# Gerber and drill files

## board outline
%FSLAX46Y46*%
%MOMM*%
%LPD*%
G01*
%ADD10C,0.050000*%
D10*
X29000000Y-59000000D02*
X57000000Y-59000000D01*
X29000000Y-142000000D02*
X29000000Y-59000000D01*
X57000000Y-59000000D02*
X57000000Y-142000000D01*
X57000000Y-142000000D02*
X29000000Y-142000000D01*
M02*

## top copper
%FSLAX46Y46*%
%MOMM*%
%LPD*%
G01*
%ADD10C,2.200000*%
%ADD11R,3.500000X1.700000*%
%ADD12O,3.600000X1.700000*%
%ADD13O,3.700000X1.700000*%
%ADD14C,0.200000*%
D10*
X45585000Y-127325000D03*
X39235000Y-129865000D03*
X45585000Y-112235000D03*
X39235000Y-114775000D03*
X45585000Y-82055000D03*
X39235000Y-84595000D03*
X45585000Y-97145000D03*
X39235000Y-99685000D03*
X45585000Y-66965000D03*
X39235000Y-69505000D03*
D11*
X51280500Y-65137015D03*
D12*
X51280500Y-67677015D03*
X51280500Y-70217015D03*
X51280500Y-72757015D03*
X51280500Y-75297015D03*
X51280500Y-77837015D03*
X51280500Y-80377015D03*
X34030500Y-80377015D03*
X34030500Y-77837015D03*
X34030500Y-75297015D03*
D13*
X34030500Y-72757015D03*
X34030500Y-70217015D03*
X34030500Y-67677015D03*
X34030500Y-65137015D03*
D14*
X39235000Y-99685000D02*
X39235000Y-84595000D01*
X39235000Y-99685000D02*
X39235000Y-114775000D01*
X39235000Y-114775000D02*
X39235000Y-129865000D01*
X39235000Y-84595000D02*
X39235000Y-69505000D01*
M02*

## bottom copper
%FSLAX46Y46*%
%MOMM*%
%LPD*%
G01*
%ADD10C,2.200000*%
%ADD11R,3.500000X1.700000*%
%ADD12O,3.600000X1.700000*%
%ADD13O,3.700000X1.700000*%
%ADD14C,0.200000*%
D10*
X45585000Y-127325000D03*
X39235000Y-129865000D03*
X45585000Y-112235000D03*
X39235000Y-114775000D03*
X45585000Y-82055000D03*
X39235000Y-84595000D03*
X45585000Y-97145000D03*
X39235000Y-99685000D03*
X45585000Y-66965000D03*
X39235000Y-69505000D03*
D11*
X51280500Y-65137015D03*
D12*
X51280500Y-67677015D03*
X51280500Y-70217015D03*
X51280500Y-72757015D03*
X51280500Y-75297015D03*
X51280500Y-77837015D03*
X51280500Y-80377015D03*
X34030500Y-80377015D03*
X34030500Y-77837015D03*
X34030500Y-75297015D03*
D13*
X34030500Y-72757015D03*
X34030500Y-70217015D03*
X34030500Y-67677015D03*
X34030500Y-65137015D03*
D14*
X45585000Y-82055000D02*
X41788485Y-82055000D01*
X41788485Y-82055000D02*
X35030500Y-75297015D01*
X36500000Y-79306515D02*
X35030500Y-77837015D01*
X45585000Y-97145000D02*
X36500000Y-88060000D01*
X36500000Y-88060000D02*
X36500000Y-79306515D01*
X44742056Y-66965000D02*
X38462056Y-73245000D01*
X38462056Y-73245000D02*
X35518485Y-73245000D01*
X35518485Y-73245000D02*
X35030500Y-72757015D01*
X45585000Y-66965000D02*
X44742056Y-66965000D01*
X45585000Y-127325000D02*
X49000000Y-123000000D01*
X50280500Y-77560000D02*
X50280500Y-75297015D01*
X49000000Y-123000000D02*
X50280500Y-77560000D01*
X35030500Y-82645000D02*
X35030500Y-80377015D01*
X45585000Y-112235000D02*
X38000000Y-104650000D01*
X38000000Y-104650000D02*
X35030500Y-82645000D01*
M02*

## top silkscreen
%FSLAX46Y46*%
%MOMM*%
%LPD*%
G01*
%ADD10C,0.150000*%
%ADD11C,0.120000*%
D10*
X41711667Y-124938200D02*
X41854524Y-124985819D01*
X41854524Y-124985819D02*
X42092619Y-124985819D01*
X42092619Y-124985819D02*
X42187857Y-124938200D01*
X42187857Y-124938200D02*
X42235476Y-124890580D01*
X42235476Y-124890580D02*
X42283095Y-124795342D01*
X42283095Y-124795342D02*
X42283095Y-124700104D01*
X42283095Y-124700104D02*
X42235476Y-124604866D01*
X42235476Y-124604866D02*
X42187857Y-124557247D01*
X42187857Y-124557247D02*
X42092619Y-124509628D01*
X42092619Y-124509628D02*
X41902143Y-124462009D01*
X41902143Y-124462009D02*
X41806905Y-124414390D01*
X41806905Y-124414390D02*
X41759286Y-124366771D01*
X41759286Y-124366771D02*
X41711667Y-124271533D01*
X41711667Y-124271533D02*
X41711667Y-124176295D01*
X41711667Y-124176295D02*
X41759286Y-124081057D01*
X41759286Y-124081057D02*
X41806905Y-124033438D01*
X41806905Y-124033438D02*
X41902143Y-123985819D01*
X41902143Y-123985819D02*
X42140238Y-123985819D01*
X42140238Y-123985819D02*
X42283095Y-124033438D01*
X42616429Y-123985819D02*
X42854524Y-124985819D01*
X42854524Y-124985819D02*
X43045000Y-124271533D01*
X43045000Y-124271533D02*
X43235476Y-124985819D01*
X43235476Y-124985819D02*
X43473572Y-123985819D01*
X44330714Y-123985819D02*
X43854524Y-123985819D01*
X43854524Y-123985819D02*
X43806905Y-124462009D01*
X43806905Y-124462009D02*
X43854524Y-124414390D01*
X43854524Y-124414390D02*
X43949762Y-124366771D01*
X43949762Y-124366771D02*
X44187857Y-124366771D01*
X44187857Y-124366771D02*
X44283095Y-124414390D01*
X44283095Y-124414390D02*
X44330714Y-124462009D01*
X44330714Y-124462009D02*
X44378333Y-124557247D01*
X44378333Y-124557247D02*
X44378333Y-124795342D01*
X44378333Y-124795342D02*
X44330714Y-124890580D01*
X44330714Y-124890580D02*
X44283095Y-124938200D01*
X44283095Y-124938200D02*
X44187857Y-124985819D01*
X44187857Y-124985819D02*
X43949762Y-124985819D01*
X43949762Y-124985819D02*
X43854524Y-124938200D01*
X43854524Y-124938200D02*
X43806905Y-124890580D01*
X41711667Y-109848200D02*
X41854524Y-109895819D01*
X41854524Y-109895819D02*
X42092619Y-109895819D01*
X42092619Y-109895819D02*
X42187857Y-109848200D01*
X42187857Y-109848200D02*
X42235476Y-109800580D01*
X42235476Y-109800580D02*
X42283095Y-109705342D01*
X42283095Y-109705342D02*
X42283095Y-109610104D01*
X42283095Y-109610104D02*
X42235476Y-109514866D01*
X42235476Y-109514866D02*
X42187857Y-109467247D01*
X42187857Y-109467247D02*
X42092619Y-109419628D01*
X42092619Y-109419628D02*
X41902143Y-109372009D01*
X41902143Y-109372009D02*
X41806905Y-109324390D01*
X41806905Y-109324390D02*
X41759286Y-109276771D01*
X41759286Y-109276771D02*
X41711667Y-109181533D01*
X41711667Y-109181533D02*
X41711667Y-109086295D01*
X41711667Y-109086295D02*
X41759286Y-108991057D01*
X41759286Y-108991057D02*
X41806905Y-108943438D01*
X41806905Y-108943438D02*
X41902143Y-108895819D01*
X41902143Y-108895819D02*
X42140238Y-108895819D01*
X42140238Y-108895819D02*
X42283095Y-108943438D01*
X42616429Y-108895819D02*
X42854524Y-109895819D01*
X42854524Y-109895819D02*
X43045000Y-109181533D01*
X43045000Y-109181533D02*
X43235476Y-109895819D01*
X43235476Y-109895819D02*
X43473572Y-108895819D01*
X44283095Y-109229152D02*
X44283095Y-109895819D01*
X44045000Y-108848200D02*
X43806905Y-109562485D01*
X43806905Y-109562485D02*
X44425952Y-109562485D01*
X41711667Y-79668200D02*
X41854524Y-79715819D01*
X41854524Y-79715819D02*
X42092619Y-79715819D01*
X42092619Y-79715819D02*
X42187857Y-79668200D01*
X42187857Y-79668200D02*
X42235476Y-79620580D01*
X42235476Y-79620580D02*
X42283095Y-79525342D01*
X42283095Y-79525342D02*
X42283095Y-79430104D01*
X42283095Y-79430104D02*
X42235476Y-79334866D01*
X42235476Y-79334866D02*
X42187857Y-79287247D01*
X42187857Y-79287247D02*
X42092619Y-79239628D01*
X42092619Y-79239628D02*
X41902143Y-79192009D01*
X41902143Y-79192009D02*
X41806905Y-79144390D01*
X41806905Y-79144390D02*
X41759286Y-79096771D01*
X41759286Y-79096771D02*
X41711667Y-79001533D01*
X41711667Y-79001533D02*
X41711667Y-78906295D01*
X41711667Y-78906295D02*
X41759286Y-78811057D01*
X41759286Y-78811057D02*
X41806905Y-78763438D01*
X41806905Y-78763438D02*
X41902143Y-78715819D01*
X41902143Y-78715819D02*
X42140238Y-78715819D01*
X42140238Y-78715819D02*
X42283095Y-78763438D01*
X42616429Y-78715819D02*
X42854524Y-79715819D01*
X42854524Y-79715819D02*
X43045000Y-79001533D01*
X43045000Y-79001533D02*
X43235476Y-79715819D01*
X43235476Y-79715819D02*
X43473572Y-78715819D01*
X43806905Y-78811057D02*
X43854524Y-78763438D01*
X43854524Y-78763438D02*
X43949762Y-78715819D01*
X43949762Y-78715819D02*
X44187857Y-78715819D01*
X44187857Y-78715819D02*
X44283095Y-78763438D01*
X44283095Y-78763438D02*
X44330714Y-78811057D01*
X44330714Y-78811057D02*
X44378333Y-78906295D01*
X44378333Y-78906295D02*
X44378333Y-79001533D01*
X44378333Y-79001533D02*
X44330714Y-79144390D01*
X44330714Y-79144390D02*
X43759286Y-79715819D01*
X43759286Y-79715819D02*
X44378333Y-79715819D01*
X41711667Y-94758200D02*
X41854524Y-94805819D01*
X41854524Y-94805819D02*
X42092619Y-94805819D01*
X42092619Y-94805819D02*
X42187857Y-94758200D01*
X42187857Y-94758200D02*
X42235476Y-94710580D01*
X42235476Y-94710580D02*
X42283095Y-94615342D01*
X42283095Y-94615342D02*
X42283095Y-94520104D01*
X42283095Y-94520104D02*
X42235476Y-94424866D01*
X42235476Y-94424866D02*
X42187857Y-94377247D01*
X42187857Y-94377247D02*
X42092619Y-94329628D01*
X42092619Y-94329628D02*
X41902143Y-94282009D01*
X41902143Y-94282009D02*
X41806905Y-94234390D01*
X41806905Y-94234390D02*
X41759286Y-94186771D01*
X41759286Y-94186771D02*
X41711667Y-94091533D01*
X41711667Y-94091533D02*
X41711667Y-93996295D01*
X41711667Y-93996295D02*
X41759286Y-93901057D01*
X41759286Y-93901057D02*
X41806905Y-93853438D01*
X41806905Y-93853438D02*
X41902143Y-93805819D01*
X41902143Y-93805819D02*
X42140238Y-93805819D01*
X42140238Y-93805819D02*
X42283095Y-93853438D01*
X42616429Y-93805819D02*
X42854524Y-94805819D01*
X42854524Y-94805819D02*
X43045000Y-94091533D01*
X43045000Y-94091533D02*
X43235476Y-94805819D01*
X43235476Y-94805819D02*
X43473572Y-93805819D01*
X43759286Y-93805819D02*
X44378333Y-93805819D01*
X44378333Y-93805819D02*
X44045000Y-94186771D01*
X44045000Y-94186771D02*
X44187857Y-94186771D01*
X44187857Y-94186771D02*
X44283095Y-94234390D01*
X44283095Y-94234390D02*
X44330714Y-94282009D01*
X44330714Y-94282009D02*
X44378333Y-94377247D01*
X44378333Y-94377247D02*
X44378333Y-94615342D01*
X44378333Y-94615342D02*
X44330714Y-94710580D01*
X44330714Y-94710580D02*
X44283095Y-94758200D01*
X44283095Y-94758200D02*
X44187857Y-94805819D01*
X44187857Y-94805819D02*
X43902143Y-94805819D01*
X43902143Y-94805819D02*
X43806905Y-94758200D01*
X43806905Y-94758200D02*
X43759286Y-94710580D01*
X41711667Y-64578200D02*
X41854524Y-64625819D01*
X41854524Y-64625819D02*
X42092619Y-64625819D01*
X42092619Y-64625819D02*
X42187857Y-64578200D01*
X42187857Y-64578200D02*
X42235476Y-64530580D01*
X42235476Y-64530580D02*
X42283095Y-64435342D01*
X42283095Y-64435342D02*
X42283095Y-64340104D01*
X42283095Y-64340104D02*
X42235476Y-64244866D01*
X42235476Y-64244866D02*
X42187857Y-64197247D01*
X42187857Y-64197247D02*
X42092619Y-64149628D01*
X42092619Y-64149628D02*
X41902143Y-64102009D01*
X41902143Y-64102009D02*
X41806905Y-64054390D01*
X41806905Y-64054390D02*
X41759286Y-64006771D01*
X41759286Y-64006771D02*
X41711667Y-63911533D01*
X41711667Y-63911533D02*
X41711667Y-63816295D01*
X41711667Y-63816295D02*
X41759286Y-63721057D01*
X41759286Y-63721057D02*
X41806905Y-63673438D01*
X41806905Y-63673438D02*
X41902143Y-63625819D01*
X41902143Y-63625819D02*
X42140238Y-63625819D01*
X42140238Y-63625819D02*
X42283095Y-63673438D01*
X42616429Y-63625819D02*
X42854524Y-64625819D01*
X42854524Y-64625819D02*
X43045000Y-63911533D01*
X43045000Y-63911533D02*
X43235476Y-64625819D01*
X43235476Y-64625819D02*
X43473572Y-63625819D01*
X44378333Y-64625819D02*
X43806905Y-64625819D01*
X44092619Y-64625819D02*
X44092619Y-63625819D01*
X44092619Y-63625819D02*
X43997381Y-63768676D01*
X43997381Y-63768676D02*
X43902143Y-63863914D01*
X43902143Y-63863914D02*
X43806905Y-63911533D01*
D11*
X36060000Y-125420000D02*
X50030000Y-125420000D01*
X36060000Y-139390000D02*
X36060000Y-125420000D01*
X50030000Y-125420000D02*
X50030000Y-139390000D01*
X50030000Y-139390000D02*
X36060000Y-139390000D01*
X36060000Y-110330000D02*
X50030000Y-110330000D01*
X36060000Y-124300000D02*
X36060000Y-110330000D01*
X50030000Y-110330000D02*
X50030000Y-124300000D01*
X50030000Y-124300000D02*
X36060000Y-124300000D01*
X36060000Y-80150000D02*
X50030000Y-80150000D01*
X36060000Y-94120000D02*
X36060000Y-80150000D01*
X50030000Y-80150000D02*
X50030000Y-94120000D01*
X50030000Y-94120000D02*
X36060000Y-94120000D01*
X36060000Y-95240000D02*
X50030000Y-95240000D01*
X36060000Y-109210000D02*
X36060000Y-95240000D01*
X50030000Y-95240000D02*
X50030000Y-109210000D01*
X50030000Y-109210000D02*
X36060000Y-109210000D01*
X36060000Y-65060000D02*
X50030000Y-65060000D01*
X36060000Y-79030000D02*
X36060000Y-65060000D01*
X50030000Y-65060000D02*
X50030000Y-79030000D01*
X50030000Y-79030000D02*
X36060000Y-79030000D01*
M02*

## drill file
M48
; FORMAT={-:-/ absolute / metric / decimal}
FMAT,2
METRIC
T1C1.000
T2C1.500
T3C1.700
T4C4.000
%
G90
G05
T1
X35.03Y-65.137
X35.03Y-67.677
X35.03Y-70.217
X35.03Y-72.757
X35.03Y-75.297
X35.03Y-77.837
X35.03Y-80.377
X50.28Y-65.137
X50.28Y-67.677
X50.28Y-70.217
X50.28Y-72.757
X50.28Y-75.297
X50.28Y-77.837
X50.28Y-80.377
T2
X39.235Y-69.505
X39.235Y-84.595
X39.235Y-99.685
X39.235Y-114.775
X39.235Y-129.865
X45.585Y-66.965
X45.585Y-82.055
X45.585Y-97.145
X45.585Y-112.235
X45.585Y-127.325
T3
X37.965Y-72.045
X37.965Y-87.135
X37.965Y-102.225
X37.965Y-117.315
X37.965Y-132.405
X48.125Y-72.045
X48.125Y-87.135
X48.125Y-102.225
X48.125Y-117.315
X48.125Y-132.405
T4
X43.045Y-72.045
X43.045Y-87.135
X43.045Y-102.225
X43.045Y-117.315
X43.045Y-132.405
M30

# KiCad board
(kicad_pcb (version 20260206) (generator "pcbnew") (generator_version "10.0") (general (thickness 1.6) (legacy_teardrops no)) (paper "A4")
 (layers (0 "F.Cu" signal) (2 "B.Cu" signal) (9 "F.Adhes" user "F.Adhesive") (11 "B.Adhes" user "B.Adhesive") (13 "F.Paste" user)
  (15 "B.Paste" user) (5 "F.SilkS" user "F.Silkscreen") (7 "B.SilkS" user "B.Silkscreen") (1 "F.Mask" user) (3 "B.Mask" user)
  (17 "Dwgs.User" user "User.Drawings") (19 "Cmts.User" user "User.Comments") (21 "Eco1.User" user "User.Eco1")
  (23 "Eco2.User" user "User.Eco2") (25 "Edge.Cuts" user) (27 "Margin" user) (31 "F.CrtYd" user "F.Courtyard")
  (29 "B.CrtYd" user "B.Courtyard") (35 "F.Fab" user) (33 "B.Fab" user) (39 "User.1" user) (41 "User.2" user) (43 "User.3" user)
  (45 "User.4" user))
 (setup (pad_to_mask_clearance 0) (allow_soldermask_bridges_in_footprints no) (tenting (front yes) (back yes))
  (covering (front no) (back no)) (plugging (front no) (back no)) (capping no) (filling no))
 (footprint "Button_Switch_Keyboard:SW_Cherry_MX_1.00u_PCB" (layer "F.Cu") (at 45.585 127.325)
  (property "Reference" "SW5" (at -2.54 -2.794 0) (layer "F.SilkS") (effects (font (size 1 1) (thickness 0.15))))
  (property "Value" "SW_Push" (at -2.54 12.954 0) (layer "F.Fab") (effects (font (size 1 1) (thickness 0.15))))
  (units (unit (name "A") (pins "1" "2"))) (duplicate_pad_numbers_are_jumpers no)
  (fp_line (start -9.525 -1.905) (end 4.445 -1.905) (stroke (width 0.12) (type solid)) (layer "F.SilkS"))
  (fp_line (start -9.525 12.065) (end -9.525 -1.905) (stroke (width 0.12) (type solid)) (layer "F.SilkS"))
  (fp_line (start 4.445 -1.905) (end 4.445 12.065) (stroke (width 0.12) (type solid)) (layer "F.SilkS"))
  (fp_line (start 4.445 12.065) (end -9.525 12.065) (stroke (width 0.12) (type solid)) (layer "F.SilkS"))
  (pad "" np_thru_hole circle (at -7.62 5.08) (size 1.7 1.7) (drill 1.7) (layers "*.Cu" "*.Mask"))
  (pad "" np_thru_hole circle (at -2.54 5.08) (size 4 4) (drill 4) (layers "*.Cu" "*.Mask"))
  (pad "" np_thru_hole circle (at 2.54 5.08) (size 1.7 1.7) (drill 1.7) (layers "*.Cu" "*.Mask"))
  (pad "1" thru_hole circle (at 0 0) (size 2.2 2.2) (drill 1.5) (layers "*.Cu" "*.Mask") (remove_unused_layers no)
   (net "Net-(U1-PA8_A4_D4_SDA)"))
  (pad "2" thru_hole circle (at -6.35 2.54) (size 2.2 2.2) (drill 1.5) (layers "*.Cu" "*.Mask") (remove_unused_layers no) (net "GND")))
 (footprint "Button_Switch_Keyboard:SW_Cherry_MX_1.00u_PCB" (layer "F.Cu") (at 45.585 112.235)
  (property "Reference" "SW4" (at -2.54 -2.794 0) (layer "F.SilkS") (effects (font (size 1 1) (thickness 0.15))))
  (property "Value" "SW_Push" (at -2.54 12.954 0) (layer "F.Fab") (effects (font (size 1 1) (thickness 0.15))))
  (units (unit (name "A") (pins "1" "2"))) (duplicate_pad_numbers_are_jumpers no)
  (fp_line (start -9.525 -1.905) (end 4.445 -1.905) (stroke (width 0.12) (type solid)) (layer "F.SilkS"))
  (fp_line (start -9.525 12.065) (end -9.525 -1.905) (stroke (width 0.12) (type solid)) (layer "F.SilkS"))
  (fp_line (start 4.445 -1.905) (end 4.445 12.065) (stroke (width 0.12) (type solid)) (layer "F.SilkS"))
  (fp_line (start 4.445 12.065) (end -9.525 12.065) (stroke (width 0.12) (type solid)) (layer "F.SilkS"))
  (pad "" np_thru_hole circle (at -7.62 5.08) (size 1.7 1.7) (drill 1.7) (layers "*.Cu" "*.Mask"))
  (pad "" np_thru_hole circle (at -2.54 5.08) (size 4 4) (drill 4) (layers "*.Cu" "*.Mask"))
  (pad "" np_thru_hole circle (at 2.54 5.08) (size 1.7 1.7) (drill 1.7) (layers "*.Cu" "*.Mask"))
  (pad "1" thru_hole circle (at 0 0) (size 2.2 2.2) (drill 1.5) (layers "*.Cu" "*.Mask") (remove_unused_layers no)
   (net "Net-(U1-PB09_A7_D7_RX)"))
  (pad "2" thru_hole circle (at -6.35 2.54) (size 2.2 2.2) (drill 1.5) (layers "*.Cu" "*.Mask") (remove_unused_layers no) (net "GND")))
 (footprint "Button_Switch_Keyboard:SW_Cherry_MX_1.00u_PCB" (layer "F.Cu") (at 45.585 82.055)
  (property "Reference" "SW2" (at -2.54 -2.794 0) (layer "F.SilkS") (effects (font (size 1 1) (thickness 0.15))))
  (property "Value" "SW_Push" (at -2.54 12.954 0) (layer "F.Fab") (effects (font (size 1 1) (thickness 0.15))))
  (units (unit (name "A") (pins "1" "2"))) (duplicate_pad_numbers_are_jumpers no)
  (fp_line (start -9.525 -1.905) (end 4.445 -1.905) (stroke (width 0.12) (type solid)) (layer "F.SilkS"))
  (fp_line (start -9.525 12.065) (end -9.525 -1.905) (stroke (width 0.12) (type solid)) (layer "F.SilkS"))
  (fp_line (start 4.445 -1.905) (end 4.445 12.065) (stroke (width 0.12) (type solid)) (layer "F.SilkS"))
  (fp_line (start 4.445 12.065) (end -9.525 12.065) (stroke (width 0.12) (type solid)) (layer "F.SilkS"))
  (pad "" np_thru_hole circle (at -7.62 5.08) (size 1.7 1.7) (drill 1.7) (layers "*.Cu" "*.Mask"))
  (pad "" np_thru_hole circle (at -2.54 5.08) (size 4 4) (drill 4) (layers "*.Cu" "*.Mask"))
  (pad "" np_thru_hole circle (at 2.54 5.08) (size 1.7 1.7) (drill 1.7) (layers "*.Cu" "*.Mask"))
  (pad "1" thru_hole circle (at 0 0) (size 2.2 2.2) (drill 1.5) (layers "*.Cu" "*.Mask") (remove_unused_layers no)
   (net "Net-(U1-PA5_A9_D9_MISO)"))
  (pad "2" thru_hole circle (at -6.35 2.54) (size 2.2 2.2) (drill 1.5) (layers "*.Cu" "*.Mask") (remove_unused_layers no) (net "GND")))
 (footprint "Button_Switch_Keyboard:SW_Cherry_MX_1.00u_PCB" (layer "F.Cu") (at 45.585 97.145)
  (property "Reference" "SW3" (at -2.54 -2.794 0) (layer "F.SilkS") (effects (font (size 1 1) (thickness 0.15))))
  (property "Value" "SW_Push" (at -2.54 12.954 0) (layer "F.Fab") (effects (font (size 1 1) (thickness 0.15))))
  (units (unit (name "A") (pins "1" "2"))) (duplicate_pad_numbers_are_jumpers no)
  (fp_line (start -9.525 -1.905) (end 4.445 -1.905) (stroke (width 0.12) (type solid)) (layer "F.SilkS"))
  (fp_line (start -9.525 12.065) (end -9.525 -1.905) (stroke (width 0.12) (type solid)) (layer "F.SilkS"))
  (fp_line (start 4.445 -1.905) (end 4.445 12.065) (stroke (width 0.12) (type solid)) (layer "F.SilkS"))
  (fp_line (start 4.445 12.065) (end -9.525 12.065) (stroke (width 0.12) (type solid)) (layer "F.SilkS"))
  (pad "" np_thru_hole circle (at -7.62 5.08) (size 1.7 1.7) (drill 1.7) (layers "*.Cu" "*.Mask"))
  (pad "" np_thru_hole circle (at -2.54 5.08) (size 4 4) (drill 4) (layers "*.Cu" "*.Mask"))
  (pad "" np_thru_hole circle (at 2.54 5.08) (size 1.7 1.7) (drill 1.7) (layers "*.Cu" "*.Mask"))
  (pad "1" thru_hole circle (at 0 0) (size 2.2 2.2) (drill 1.5) (layers "*.Cu" "*.Mask") (remove_unused_layers no)
   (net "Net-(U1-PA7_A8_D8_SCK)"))
  (pad "2" thru_hole circle (at -6.35 2.54) (size 2.2 2.2) (drill 1.5) (layers "*.Cu" "*.Mask") (remove_unused_layers no) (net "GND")))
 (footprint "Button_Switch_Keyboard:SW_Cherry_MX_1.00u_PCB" (layer "F.Cu") (at 45.585 66.965)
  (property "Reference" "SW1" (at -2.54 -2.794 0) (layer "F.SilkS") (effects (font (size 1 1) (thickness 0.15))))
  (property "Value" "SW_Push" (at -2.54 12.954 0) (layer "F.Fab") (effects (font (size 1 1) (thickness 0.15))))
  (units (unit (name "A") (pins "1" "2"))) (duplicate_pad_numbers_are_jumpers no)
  (fp_line (start -9.525 -1.905) (end 4.445 -1.905) (stroke (width 0.12) (type solid)) (layer "F.SilkS"))
  (fp_line (start -9.525 12.065) (end -9.525 -1.905) (stroke (width 0.12) (type solid)) (layer "F.SilkS"))
  (fp_line (start 4.445 -1.905) (end 4.445 12.065) (stroke (width 0.12) (type solid)) (layer "F.SilkS"))
  (fp_line (start 4.445 12.065) (end -9.525 12.065) (stroke (width 0.12) (type solid)) (layer "F.SilkS"))
  (pad "" np_thru_hole circle (at -7.62 5.08) (size 1.7 1.7) (drill 1.7) (layers "*.Cu" "*.Mask"))
  (pad "" np_thru_hole circle (at -2.54 5.08) (size 4 4) (drill 4) (layers "*.Cu" "*.Mask"))
  (pad "" np_thru_hole circle (at 2.54 5.08) (size 1.7 1.7) (drill 1.7) (layers "*.Cu" "*.Mask"))
  (pad "1" thru_hole circle (at 0 0) (size 2.2 2.2) (drill 1.5) (layers "*.Cu" "*.Mask") (remove_unused_layers no)
   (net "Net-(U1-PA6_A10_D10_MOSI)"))
  (pad "2" thru_hole circle (at -6.35 2.54) (size 2.2 2.2) (drill 1.5) (layers "*.Cu" "*.Mask") (remove_unused_layers no) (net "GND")))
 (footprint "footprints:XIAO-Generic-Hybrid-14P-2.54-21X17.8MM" (layer "B.Cu") (at 42.6555 72.757015 180)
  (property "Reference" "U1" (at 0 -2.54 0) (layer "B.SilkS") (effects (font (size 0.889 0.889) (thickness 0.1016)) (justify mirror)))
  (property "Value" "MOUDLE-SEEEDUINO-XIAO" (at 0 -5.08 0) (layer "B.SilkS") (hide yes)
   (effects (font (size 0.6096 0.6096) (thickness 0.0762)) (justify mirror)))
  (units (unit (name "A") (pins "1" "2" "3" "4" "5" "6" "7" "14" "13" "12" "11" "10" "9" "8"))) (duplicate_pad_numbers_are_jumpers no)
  (pad "1" thru_hole rect (at -7.625 7.62 180) (size 3.5 1.7) (drill 1 (offset -1 0)) (layers "*.Cu" "*.Mask") (remove_unused_layers no)
   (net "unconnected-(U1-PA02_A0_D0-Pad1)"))
  (pad "2" thru_hole oval (at -7.625 5.08 180) (size 3.6 1.7) (drill 1 (offset -1 0)) (layers "*.Cu" "*.Mask") (remove_unused_layers no)
   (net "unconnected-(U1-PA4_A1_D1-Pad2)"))
  (pad "3" thru_hole oval (at -7.625 2.54 180) (size 3.6 1.7) (drill 1 (offset -1 0)) (layers "*.Cu" "*.Mask") (remove_unused_layers no)
   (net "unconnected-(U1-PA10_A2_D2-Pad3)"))
  (pad "4" thru_hole oval (at -7.625 0 180) (size 3.6 1.7) (drill 1 (offset -1 0)) (layers "*.Cu" "*.Mask") (remove_unused_layers no)
   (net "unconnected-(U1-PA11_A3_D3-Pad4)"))
  (pad "5" thru_hole oval (at -7.625 -2.54 180) (size 3.6 1.7) (drill 1 (offset -1 0)) (layers "*.Cu" "*.Mask") (remove_unused_layers no)
   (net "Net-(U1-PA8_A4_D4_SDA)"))
  (pad "6" thru_hole oval (at -7.625 -5.08) (size 3.6 1.7) (drill 1 (offset 1 0)) (layers "*.Cu" "*.Mask") (remove_unused_layers no)
   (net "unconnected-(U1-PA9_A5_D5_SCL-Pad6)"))
  (pad "7" thru_hole oval (at -7.625 -7.62 180) (size 3.6 1.7) (drill 1 (offset -1 0)) (layers "*.Cu" "*.Mask") (remove_unused_layers no)
   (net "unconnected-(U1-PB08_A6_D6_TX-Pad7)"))
  (pad "8" thru_hole oval (at 7.625 -7.62 180) (size 3.6 1.7) (drill 1 (offset 1 0)) (layers "*.Cu" "*.Mask") (remove_unused_layers no)
   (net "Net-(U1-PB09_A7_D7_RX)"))
  (pad "9" thru_hole oval (at 7.625 -5.08 180) (size 3.6 1.7) (drill 1 (offset 1 0)) (layers "*.Cu" "*.Mask") (remove_unused_layers no)
   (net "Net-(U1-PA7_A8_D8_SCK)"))
  (pad "10" thru_hole oval (at 7.625 -2.54 180) (size 3.6 1.7) (drill 1 (offset 1 0)) (layers "*.Cu" "*.Mask") (remove_unused_layers no)
   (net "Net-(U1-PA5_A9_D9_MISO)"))
  (pad "11" thru_hole oval (at 7.625 0 180) (size 3.7 1.7) (drill 1 (offset 1 0)) (layers "*.Cu" "*.Mask") (remove_unused_layers no)
   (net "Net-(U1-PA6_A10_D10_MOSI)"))
  (pad "12" thru_hole oval (at 7.625 2.54 180) (size 3.7 1.7) (drill 1 (offset 1 0)) (layers "*.Cu" "*.Mask") (remove_unused_layers no)
   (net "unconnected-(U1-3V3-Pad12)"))
  (pad "13" thru_hole oval (at 7.625 5.08 180) (size 3.7 1.7) (drill 1 (offset 1 0)) (layers "*.Cu" "*.Mask") (remove_unused_layers no)
   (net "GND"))
  (pad "14" thru_hole oval (at 7.625 7.62 180) (size 3.7 1.7) (drill 1 (offset 1 0)) (layers "*.Cu" "*.Mask") (remove_unused_layers no)
   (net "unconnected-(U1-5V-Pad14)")))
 (gr_line (start 29 59) (end 57 59) (stroke (width 0.05) (type default)) (layer "Edge.Cuts"))
 (gr_line (start 29 142) (end 29 59) (stroke (width 0.05) (type default)) (layer "Edge.Cuts"))
 (gr_line (start 57 59) (end 57 142) (stroke (width 0.05) (type default)) (layer "Edge.Cuts"))
 (gr_line (start 57 142) (end 29 142) (stroke (width 0.05) (type default)) (layer "Edge.Cuts"))
 (segment (start 45.585 82.055) (end 41.788485 82.055) (width 0.2) (layer "B.Cu") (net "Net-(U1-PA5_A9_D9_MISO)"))
 (segment (start 41.788485 82.055) (end 35.0305 75.297015) (width 0.2) (layer "B.Cu") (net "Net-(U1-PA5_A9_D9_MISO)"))
 (segment (start 39.235 99.685) (end 39.235 84.595) (width 0.2) (layer "F.Cu") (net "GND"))
 (segment (start 39.235 99.685) (end 39.235 114.775) (width 0.2) (layer "F.Cu") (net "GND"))
 (segment (start 39.235 114.775) (end 39.235 129.865) (width 0.2) (layer "F.Cu") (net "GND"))
 (segment (start 39.235 84.595) (end 39.235 69.505) (width 0.2) (layer "F.Cu") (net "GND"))
 (segment (start 36.5 79.306515) (end 35.0305 77.837015) (width 0.2) (layer "B.Cu") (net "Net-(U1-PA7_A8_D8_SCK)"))
 (segment (start 45.585 97.145) (end 36.5 88.06) (width 0.2) (layer "B.Cu") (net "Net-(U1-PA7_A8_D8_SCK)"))
 (segment (start 36.5 88.06) (end 36.5 79.306515) (width 0.2) (layer "B.Cu") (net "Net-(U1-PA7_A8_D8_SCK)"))
 (segment (start 44.742056 66.965) (end 38.462056 73.245) (width 0.2) (layer "B.Cu") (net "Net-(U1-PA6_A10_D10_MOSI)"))
 (segment (start 38.462056 73.245) (end 35.518485 73.245) (width 0.2) (layer "B.Cu") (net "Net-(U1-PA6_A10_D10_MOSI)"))
 (segment (start 35.518485 73.245) (end 35.0305 72.757015) (width 0.2) (layer "B.Cu") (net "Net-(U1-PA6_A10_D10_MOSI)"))
 (segment (start 45.585 66.965) (end 44.742056 66.965) (width 0.2) (layer "B.Cu") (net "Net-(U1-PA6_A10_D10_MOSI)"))
 (segment (start 45.585 127.325) (end 49 123) (width 0.2) (layer "B.Cu") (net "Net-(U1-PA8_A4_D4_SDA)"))
 (segment (start 50.2805 77.56) (end 50.2805 75.297015) (width 0.2) (layer "B.Cu") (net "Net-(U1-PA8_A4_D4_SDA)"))
 (segment (start 49 123) (end 50.2805 77.56) (width 0.2) (layer "B.Cu") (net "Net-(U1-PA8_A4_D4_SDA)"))
 (segment (start 35.0305 82.645) (end 35.0305 80.377015) (width 0.2) (layer "B.Cu") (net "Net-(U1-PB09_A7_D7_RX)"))
 (segment (start 45.585 112.235) (end 38 104.65) (width 0.2) (layer "B.Cu") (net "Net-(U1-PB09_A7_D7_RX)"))
 (segment (start 38 104.65) (end 35.0305 82.645) (width 0.2) (layer "B.Cu") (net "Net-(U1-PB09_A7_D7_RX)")))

